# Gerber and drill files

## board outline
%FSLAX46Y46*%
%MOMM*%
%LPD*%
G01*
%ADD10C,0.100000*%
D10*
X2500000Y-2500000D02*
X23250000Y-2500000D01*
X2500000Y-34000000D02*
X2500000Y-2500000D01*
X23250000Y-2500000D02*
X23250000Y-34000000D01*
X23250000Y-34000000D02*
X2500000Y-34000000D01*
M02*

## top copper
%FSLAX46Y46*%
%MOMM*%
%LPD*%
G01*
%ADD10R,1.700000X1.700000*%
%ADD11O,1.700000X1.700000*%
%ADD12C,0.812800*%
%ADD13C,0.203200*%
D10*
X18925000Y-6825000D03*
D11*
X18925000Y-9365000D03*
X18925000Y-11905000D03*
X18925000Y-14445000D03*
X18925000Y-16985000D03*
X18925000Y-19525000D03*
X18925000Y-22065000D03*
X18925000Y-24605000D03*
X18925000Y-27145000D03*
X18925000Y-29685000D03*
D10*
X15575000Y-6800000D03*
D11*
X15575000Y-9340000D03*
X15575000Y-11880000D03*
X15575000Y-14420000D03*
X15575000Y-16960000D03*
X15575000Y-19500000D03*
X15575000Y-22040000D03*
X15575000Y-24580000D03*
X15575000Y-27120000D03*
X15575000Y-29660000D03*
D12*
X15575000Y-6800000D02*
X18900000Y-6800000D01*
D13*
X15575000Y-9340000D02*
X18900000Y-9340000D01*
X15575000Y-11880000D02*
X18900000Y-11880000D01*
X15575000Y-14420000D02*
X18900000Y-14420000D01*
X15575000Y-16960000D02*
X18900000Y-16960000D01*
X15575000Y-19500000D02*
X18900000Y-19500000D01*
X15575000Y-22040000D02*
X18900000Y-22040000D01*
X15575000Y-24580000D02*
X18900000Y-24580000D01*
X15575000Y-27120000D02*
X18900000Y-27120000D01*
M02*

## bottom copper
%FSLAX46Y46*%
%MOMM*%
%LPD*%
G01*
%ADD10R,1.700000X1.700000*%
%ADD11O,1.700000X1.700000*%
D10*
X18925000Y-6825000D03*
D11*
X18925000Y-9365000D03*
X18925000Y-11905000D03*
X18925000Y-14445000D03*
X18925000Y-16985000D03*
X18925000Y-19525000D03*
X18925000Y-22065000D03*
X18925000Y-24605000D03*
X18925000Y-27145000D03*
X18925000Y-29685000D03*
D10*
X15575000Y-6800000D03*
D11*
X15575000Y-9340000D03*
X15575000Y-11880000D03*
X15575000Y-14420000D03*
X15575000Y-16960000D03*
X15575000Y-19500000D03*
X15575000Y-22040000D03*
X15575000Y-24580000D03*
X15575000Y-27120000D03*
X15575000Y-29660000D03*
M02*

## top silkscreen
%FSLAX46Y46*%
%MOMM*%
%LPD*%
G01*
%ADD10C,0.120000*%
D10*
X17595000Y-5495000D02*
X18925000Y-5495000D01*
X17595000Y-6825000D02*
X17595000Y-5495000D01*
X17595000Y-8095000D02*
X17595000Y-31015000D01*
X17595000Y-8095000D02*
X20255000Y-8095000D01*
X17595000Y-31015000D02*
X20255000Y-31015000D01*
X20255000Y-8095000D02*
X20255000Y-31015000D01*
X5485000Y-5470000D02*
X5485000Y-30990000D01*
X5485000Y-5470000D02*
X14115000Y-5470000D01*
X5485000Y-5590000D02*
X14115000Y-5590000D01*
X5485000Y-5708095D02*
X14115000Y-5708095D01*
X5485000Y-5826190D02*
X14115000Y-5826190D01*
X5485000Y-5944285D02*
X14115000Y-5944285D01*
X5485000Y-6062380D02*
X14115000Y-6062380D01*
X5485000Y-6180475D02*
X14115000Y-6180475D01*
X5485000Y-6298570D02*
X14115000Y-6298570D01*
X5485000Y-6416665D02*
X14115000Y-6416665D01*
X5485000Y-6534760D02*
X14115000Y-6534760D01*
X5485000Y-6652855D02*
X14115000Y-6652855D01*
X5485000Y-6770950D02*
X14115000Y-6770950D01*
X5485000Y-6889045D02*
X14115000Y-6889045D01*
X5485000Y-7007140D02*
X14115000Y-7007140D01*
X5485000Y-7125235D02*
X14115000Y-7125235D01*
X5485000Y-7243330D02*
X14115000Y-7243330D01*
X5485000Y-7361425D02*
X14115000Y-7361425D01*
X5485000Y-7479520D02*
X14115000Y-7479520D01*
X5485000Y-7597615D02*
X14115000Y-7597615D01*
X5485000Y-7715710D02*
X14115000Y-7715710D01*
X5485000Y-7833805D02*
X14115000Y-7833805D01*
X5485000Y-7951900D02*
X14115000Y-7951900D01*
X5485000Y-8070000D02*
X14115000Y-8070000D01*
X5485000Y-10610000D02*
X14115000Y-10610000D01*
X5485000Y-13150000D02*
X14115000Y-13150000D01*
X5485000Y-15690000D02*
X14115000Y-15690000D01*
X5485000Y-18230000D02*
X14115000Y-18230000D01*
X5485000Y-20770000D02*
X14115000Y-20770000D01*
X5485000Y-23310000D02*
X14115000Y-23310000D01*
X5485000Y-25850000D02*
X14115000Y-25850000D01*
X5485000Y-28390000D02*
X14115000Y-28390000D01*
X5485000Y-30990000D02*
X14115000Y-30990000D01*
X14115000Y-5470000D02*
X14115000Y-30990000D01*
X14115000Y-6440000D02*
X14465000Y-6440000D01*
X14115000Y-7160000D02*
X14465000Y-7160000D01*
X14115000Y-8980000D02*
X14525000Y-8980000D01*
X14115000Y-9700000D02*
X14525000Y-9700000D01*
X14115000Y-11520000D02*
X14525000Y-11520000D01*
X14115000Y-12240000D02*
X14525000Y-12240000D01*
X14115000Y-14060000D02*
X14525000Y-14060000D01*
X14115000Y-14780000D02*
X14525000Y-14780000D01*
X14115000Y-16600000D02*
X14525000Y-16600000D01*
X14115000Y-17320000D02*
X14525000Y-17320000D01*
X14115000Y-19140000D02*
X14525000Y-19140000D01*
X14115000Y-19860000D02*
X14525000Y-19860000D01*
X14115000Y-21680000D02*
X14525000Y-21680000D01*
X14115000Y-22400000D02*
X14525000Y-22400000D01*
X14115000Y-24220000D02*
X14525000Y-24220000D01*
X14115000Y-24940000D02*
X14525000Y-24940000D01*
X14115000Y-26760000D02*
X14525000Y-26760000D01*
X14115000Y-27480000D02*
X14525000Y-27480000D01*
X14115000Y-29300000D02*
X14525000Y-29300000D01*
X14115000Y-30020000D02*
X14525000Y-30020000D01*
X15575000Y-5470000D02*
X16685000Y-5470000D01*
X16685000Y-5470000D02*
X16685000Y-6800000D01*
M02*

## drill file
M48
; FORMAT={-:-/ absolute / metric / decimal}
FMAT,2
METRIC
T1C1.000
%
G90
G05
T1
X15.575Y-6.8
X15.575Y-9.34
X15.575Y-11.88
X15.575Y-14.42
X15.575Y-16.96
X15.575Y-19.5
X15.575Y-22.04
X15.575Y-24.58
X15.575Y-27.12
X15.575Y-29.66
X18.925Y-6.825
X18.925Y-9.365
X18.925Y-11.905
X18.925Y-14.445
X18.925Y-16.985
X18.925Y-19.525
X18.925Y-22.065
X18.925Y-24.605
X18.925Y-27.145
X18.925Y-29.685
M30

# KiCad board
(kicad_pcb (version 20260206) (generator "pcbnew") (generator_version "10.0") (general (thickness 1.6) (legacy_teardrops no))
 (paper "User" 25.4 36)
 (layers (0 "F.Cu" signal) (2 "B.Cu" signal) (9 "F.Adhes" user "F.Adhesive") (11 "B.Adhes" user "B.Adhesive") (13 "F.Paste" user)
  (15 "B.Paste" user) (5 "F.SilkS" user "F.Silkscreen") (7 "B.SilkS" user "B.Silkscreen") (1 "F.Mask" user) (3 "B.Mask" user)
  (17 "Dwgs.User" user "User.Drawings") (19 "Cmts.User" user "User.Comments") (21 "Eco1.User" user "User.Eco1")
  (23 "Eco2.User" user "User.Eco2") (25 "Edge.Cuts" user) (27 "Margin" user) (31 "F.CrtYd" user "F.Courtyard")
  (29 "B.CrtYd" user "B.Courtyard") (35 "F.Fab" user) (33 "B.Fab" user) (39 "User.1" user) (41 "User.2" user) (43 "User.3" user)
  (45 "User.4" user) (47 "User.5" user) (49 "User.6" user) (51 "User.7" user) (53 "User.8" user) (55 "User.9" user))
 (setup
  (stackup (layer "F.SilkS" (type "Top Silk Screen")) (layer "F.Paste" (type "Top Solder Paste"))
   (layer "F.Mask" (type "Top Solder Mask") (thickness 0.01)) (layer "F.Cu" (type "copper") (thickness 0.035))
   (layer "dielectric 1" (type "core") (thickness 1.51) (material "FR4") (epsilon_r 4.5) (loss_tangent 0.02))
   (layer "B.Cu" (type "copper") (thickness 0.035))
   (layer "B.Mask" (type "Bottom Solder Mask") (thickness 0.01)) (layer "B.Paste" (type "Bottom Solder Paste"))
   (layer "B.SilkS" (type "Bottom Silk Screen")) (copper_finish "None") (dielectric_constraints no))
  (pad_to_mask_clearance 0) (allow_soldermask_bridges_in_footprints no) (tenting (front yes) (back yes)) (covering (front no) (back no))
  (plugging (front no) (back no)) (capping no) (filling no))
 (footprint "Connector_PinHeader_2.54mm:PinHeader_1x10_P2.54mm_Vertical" (layer "F.Cu") (at 18.925 6.825)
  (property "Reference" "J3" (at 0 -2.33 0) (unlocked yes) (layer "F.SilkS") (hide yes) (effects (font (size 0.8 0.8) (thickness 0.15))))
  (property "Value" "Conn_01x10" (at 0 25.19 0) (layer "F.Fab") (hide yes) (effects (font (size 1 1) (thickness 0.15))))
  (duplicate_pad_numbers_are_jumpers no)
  (fp_line (start -1.33 -1.33) (end 0 -1.33) (stroke (width 0.12) (type solid)) (layer "F.SilkS"))
  (fp_line (start -1.33 0) (end -1.33 -1.33) (stroke (width 0.12) (type solid)) (layer "F.SilkS"))
  (fp_line (start -1.33 1.27) (end -1.33 24.19) (stroke (width 0.12) (type solid)) (layer "F.SilkS"))
  (fp_line (start -1.33 1.27) (end 1.33 1.27) (stroke (width 0.12) (type solid)) (layer "F.SilkS"))
  (fp_line (start -1.33 24.19) (end 1.33 24.19) (stroke (width 0.12) (type solid)) (layer "F.SilkS"))
  (fp_line (start 1.33 1.27) (end 1.33 24.19) (stroke (width 0.12) (type solid)) (layer "F.SilkS"))
  (pad "1" thru_hole rect (at 0 0) (size 1.7 1.7) (drill 1) (layers "*.Cu" "*.Mask") (remove_unused_layers no) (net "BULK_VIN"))
  (pad "2" thru_hole oval (at 0 2.54) (size 1.7 1.7) (drill 1) (layers "*.Cu" "*.Mask") (remove_unused_layers no) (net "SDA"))
  (pad "3" thru_hole oval (at 0 5.08) (size 1.7 1.7) (drill 1) (layers "*.Cu" "*.Mask") (remove_unused_layers no) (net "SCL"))
  (pad "4" thru_hole oval (at 0 7.62) (size 1.7 1.7) (drill 1) (layers "*.Cu" "*.Mask") (remove_unused_layers no) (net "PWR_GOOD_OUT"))
  (pad "5" thru_hole oval (at 0 10.16) (size 1.7 1.7) (drill 1) (layers "*.Cu" "*.Mask") (remove_unused_layers no) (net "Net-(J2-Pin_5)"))
  (pad "6" thru_hole oval (at 0 12.7) (size 1.7 1.7) (drill 1) (layers "*.Cu" "*.Mask") (remove_unused_layers no) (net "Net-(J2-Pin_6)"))
  (pad "7" thru_hole oval (at 0 15.24) (size 1.7 1.7) (drill 1) (layers "*.Cu" "*.Mask") (remove_unused_layers no) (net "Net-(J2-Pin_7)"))
  (pad "8" thru_hole oval (at 0 17.78) (size 1.7 1.7) (drill 1) (layers "*.Cu" "*.Mask") (remove_unused_layers no) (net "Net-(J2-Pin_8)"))
  (pad "9" thru_hole oval (at 0 20.32) (size 1.7 1.7) (drill 1) (layers "*.Cu" "*.Mask") (remove_unused_layers no) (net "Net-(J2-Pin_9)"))
  (pad "10" thru_hole oval (at 0 22.86) (size 1.7 1.7) (drill 1) (layers "*.Cu" "*.Mask") (remove_unused_layers no) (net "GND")))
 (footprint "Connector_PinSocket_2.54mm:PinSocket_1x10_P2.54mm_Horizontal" (layer "F.Cu") (at 15.575 6.8)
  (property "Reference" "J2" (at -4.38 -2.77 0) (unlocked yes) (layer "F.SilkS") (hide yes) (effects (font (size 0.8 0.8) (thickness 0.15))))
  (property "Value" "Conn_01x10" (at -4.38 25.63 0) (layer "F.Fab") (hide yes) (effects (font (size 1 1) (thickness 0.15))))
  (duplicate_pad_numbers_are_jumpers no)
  (fp_line (start -10.09 -1.33) (end -10.09 24.19) (stroke (width 0.12) (type solid)) (layer "F.SilkS"))
  (fp_line (start -10.09 -1.33) (end -1.46 -1.33) (stroke (width 0.12) (type solid)) (layer "F.SilkS"))
  (fp_line (start -10.09 -1.21) (end -1.46 -1.21) (stroke (width 0.12) (type solid)) (layer "F.SilkS"))
  (fp_line (start -10.09 -1.091905) (end -1.46 -1.091905) (stroke (width 0.12) (type solid)) (layer "F.SilkS"))
  (fp_line (start -10.09 -0.97381) (end -1.46 -0.97381) (stroke (width 0.12) (type solid)) (layer "F.SilkS"))
  (fp_line (start -10.09 -0.855715) (end -1.46 -0.855715) (stroke (width 0.12) (type solid)) (layer "F.SilkS"))
  (fp_line (start -10.09 -0.73762) (end -1.46 -0.73762) (stroke (width 0.12) (type solid)) (layer "F.SilkS"))
  (fp_line (start -10.09 -0.619525) (end -1.46 -0.619525) (stroke (width 0.12) (type solid)) (layer "F.SilkS"))
  (fp_line (start -10.09 -0.50143) (end -1.46 -0.50143) (stroke (width 0.12) (type solid)) (layer "F.SilkS"))
  (fp_line (start -10.09 -0.383335) (end -1.46 -0.383335) (stroke (width 0.12) (type solid)) (layer "F.SilkS"))
  (fp_line (start -10.09 -0.26524) (end -1.46 -0.26524) (stroke (width 0.12) (type solid)) (layer "F.SilkS"))
  (fp_line (start -10.09 -0.147145) (end -1.46 -0.147145) (stroke (width 0.12) (type solid)) (layer "F.SilkS"))
  (fp_line (start -10.09 -0.02905) (end -1.46 -0.02905) (stroke (width 0.12) (type solid)) (layer "F.SilkS"))
  (fp_line (start -10.09 0.089045) (end -1.46 0.089045) (stroke (width 0.12) (type solid)) (layer "F.SilkS"))
  (fp_line (start -10.09 0.20714) (end -1.46 0.20714) (stroke (width 0.12) (type solid)) (layer "F.SilkS"))
  (fp_line (start -10.09 0.325235) (end -1.46 0.325235) (stroke (width 0.12) (type solid)) (layer "F.SilkS"))
  (fp_line (start -10.09 0.44333) (end -1.46 0.44333) (stroke (width 0.12) (type solid)) (layer "F.SilkS"))
  (fp_line (start -10.09 0.561425) (end -1.46 0.561425) (stroke (width 0.12) (type solid)) (layer "F.SilkS"))
  (fp_line (start -10.09 0.67952) (end -1.46 0.67952) (stroke (width 0.12) (type solid)) (layer "F.SilkS"))
  (fp_line (start -10.09 0.797615) (end -1.46 0.797615) (stroke (width 0.12) (type solid)) (layer "F.SilkS"))
  (fp_line (start -10.09 0.91571) (end -1.46 0.91571) (stroke (width 0.12) (type solid)) (layer "F.SilkS"))
  (fp_line (start -10.09 1.033805) (end -1.46 1.033805) (stroke (width 0.12) (type solid)) (layer "F.SilkS"))
  (fp_line (start -10.09 1.1519) (end -1.46 1.1519) (stroke (width 0.12) (type solid)) (layer "F.SilkS"))
  (fp_line (start -10.09 1.27) (end -1.46 1.27) (stroke (width 0.12) (type solid)) (layer "F.SilkS"))
  (fp_line (start -10.09 3.81) (end -1.46 3.81) (stroke (width 0.12) (type solid)) (layer "F.SilkS"))
  (fp_line (start -10.09 6.35) (end -1.46 6.35) (stroke (width 0.12) (type solid)) (layer "F.SilkS"))
  (fp_line (start -10.09 8.89) (end -1.46 8.89) (stroke (width 0.12) (type solid)) (layer "F.SilkS"))
  (fp_line (start -10.09 11.43) (end -1.46 11.43) (stroke (width 0.12) (type solid)) (layer "F.SilkS"))
  (fp_line (start -10.09 13.97) (end -1.46 13.97) (stroke (width 0.12) (type solid)) (layer "F.SilkS"))
  (fp_line (start -10.09 16.51) (end -1.46 16.51) (stroke (width 0.12) (type solid)) (layer "F.SilkS"))
  (fp_line (start -10.09 19.05) (end -1.46 19.05) (stroke (width 0.12) (type solid)) (layer "F.SilkS"))
  (fp_line (start -10.09 21.59) (end -1.46 21.59) (stroke (width 0.12) (type solid)) (layer "F.SilkS"))
  (fp_line (start -10.09 24.19) (end -1.46 24.19) (stroke (width 0.12) (type solid)) (layer "F.SilkS"))
  (fp_line (start -1.46 -1.33) (end -1.46 24.19) (stroke (width 0.12) (type solid)) (layer "F.SilkS"))
  (fp_line (start -1.46 -0.36) (end -1.11 -0.36) (stroke (width 0.12) (type solid)) (layer "F.SilkS"))
  (fp_line (start -1.46 0.36) (end -1.11 0.36) (stroke (width 0.12) (type solid)) (layer "F.SilkS"))
  (fp_line (start -1.46 2.18) (end -1.05 2.18) (stroke (width 0.12) (type solid)) (layer "F.SilkS"))
  (fp_line (start -1.46 2.9) (end -1.05 2.9) (stroke (width 0.12) (type solid)) (layer "F.SilkS"))
  (fp_line (start -1.46 4.72) (end -1.05 4.72) (stroke (width 0.12) (type solid)) (layer "F.SilkS"))
  (fp_line (start -1.46 5.44) (end -1.05 5.44) (stroke (width 0.12) (type solid)) (layer "F.SilkS"))
  (fp_line (start -1.46 7.26) (end -1.05 7.26) (stroke (width 0.12) (type solid)) (layer "F.SilkS"))
  (fp_line (start -1.46 7.98) (end -1.05 7.98) (stroke (width 0.12) (type solid)) (layer "F.SilkS"))
  (fp_line (start -1.46 9.8) (end -1.05 9.8) (stroke (width 0.12) (type solid)) (layer "F.SilkS"))
  (fp_line (start -1.46 10.52) (end -1.05 10.52) (stroke (width 0.12) (type solid)) (layer "F.SilkS"))
  (fp_line (start -1.46 12.34) (end -1.05 12.34) (stroke (width 0.12) (type solid)) (layer "F.SilkS"))
  (fp_line (start -1.46 13.06) (end -1.05 13.06) (stroke (width 0.12) (type solid)) (layer "F.SilkS"))
  (fp_line (start -1.46 14.88) (end -1.05 14.88) (stroke (width 0.12) (type solid)) (layer "F.SilkS"))
  (fp_line (start -1.46 15.6) (end -1.05 15.6) (stroke (width 0.12) (type solid)) (layer "F.SilkS"))
  (fp_line (start -1.46 17.42) (end -1.05 17.42) (stroke (width 0.12) (type solid)) (layer "F.SilkS"))
  (fp_line (start -1.46 18.14) (end -1.05 18.14) (stroke (width 0.12) (type solid)) (layer "F.SilkS"))
  (fp_line (start -1.46 19.96) (end -1.05 19.96) (stroke (width 0.12) (type solid)) (layer "F.SilkS"))
  (fp_line (start -1.46 20.68) (end -1.05 20.68) (stroke (width 0.12) (type solid)) (layer "F.SilkS"))
  (fp_line (start -1.46 22.5) (end -1.05 22.5) (stroke (width 0.12) (type solid)) (layer "F.SilkS"))
  (fp_line (start -1.46 23.22) (end -1.05 23.22) (stroke (width 0.12) (type solid)) (layer "F.SilkS"))
  (fp_line (start 0 -1.33) (end 1.11 -1.33) (stroke (width 0.12) (type solid)) (layer "F.SilkS"))
  (fp_line (start 1.11 -1.33) (end 1.11 0) (stroke (width 0.12) (type solid)) (layer "F.SilkS"))
  (pad "1" thru_hole rect (at 0 0) (size 1.7 1.7) (drill 1) (layers "*.Cu" "*.Mask") (remove_unused_layers no) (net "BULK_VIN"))
  (pad "2" thru_hole oval (at 0 2.54) (size 1.7 1.7) (drill 1) (layers "*.Cu" "*.Mask") (remove_unused_layers no) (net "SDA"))
  (pad "3" thru_hole oval (at 0 5.08) (size 1.7 1.7) (drill 1) (layers "*.Cu" "*.Mask") (remove_unused_layers no) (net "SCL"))
  (pad "4" thru_hole oval (at 0 7.62) (size 1.7 1.7) (drill 1) (layers "*.Cu" "*.Mask") (remove_unused_layers no) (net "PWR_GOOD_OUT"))
  (pad "5" thru_hole oval (at 0 10.16) (size 1.7 1.7) (drill 1) (layers "*.Cu" "*.Mask") (remove_unused_layers no) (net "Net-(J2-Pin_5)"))
  (pad "6" thru_hole oval (at 0 12.7) (size 1.7 1.7) (drill 1) (layers "*.Cu" "*.Mask") (remove_unused_layers no) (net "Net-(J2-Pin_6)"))
  (pad "7" thru_hole oval (at 0 15.24) (size 1.7 1.7) (drill 1) (layers "*.Cu" "*.Mask") (remove_unused_layers no) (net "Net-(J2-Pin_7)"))
  (pad "8" thru_hole oval (at 0 17.78) (size 1.7 1.7) (drill 1) (layers "*.Cu" "*.Mask") (remove_unused_layers no) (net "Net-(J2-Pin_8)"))
  (pad "9" thru_hole oval (at 0 20.32) (size 1.7 1.7) (drill 1) (layers "*.Cu" "*.Mask") (remove_unused_layers no) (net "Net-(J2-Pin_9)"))
  (pad "10" thru_hole oval (at 0 22.86) (size 1.7 1.7) (drill 1) (layers "*.Cu" "*.Mask") (remove_unused_layers no) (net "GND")))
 (gr_line (start 2.5 2.5) (end 23.25 2.5) (stroke (width 0.1) (type default)) (layer "Edge.Cuts"))
 (gr_line (start 2.5 34) (end 2.5 2.5) (stroke (width 0.1) (type default)) (layer "Edge.Cuts"))
 (gr_line (start 23.25 2.5) (end 23.25 34) (stroke (width 0.1) (type default)) (layer "Edge.Cuts"))
 (gr_line (start 23.25 34) (end 2.5 34) (stroke (width 0.1) (type default)) (layer "Edge.Cuts"))
 (segment (start 15.575 6.8) (end 18.9 6.8) (width 0.8128) (layer "F.Cu") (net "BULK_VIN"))
 (segment (start 15.575 9.34) (end 18.9 9.34) (width 0.2032) (layer "F.Cu") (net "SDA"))
 (segment (start 15.575 11.88) (end 18.9 11.88) (width 0.2032) (layer "F.Cu") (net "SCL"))
 (segment (start 15.575 14.42) (end 18.9 14.42) (width 0.2032) (layer "F.Cu") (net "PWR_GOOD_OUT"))
 (segment (start 15.575 16.96) (end 18.9 16.96) (width 0.2032) (layer "F.Cu") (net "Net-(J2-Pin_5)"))
 (segment (start 15.575 19.5) (end 18.9 19.5) (width 0.2032) (layer "F.Cu") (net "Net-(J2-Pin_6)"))
 (segment (start 15.575 22.04) (end 18.9 22.04) (width 0.2032) (layer "F.Cu") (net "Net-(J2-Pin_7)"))
 (segment (start 15.575 24.58) (end 18.9 24.58) (width 0.2032) (layer "F.Cu") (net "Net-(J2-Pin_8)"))
 (segment (start 15.575 27.12) (end 18.9 27.12) (width 0.2032) (layer "F.Cu") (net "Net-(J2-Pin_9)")))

